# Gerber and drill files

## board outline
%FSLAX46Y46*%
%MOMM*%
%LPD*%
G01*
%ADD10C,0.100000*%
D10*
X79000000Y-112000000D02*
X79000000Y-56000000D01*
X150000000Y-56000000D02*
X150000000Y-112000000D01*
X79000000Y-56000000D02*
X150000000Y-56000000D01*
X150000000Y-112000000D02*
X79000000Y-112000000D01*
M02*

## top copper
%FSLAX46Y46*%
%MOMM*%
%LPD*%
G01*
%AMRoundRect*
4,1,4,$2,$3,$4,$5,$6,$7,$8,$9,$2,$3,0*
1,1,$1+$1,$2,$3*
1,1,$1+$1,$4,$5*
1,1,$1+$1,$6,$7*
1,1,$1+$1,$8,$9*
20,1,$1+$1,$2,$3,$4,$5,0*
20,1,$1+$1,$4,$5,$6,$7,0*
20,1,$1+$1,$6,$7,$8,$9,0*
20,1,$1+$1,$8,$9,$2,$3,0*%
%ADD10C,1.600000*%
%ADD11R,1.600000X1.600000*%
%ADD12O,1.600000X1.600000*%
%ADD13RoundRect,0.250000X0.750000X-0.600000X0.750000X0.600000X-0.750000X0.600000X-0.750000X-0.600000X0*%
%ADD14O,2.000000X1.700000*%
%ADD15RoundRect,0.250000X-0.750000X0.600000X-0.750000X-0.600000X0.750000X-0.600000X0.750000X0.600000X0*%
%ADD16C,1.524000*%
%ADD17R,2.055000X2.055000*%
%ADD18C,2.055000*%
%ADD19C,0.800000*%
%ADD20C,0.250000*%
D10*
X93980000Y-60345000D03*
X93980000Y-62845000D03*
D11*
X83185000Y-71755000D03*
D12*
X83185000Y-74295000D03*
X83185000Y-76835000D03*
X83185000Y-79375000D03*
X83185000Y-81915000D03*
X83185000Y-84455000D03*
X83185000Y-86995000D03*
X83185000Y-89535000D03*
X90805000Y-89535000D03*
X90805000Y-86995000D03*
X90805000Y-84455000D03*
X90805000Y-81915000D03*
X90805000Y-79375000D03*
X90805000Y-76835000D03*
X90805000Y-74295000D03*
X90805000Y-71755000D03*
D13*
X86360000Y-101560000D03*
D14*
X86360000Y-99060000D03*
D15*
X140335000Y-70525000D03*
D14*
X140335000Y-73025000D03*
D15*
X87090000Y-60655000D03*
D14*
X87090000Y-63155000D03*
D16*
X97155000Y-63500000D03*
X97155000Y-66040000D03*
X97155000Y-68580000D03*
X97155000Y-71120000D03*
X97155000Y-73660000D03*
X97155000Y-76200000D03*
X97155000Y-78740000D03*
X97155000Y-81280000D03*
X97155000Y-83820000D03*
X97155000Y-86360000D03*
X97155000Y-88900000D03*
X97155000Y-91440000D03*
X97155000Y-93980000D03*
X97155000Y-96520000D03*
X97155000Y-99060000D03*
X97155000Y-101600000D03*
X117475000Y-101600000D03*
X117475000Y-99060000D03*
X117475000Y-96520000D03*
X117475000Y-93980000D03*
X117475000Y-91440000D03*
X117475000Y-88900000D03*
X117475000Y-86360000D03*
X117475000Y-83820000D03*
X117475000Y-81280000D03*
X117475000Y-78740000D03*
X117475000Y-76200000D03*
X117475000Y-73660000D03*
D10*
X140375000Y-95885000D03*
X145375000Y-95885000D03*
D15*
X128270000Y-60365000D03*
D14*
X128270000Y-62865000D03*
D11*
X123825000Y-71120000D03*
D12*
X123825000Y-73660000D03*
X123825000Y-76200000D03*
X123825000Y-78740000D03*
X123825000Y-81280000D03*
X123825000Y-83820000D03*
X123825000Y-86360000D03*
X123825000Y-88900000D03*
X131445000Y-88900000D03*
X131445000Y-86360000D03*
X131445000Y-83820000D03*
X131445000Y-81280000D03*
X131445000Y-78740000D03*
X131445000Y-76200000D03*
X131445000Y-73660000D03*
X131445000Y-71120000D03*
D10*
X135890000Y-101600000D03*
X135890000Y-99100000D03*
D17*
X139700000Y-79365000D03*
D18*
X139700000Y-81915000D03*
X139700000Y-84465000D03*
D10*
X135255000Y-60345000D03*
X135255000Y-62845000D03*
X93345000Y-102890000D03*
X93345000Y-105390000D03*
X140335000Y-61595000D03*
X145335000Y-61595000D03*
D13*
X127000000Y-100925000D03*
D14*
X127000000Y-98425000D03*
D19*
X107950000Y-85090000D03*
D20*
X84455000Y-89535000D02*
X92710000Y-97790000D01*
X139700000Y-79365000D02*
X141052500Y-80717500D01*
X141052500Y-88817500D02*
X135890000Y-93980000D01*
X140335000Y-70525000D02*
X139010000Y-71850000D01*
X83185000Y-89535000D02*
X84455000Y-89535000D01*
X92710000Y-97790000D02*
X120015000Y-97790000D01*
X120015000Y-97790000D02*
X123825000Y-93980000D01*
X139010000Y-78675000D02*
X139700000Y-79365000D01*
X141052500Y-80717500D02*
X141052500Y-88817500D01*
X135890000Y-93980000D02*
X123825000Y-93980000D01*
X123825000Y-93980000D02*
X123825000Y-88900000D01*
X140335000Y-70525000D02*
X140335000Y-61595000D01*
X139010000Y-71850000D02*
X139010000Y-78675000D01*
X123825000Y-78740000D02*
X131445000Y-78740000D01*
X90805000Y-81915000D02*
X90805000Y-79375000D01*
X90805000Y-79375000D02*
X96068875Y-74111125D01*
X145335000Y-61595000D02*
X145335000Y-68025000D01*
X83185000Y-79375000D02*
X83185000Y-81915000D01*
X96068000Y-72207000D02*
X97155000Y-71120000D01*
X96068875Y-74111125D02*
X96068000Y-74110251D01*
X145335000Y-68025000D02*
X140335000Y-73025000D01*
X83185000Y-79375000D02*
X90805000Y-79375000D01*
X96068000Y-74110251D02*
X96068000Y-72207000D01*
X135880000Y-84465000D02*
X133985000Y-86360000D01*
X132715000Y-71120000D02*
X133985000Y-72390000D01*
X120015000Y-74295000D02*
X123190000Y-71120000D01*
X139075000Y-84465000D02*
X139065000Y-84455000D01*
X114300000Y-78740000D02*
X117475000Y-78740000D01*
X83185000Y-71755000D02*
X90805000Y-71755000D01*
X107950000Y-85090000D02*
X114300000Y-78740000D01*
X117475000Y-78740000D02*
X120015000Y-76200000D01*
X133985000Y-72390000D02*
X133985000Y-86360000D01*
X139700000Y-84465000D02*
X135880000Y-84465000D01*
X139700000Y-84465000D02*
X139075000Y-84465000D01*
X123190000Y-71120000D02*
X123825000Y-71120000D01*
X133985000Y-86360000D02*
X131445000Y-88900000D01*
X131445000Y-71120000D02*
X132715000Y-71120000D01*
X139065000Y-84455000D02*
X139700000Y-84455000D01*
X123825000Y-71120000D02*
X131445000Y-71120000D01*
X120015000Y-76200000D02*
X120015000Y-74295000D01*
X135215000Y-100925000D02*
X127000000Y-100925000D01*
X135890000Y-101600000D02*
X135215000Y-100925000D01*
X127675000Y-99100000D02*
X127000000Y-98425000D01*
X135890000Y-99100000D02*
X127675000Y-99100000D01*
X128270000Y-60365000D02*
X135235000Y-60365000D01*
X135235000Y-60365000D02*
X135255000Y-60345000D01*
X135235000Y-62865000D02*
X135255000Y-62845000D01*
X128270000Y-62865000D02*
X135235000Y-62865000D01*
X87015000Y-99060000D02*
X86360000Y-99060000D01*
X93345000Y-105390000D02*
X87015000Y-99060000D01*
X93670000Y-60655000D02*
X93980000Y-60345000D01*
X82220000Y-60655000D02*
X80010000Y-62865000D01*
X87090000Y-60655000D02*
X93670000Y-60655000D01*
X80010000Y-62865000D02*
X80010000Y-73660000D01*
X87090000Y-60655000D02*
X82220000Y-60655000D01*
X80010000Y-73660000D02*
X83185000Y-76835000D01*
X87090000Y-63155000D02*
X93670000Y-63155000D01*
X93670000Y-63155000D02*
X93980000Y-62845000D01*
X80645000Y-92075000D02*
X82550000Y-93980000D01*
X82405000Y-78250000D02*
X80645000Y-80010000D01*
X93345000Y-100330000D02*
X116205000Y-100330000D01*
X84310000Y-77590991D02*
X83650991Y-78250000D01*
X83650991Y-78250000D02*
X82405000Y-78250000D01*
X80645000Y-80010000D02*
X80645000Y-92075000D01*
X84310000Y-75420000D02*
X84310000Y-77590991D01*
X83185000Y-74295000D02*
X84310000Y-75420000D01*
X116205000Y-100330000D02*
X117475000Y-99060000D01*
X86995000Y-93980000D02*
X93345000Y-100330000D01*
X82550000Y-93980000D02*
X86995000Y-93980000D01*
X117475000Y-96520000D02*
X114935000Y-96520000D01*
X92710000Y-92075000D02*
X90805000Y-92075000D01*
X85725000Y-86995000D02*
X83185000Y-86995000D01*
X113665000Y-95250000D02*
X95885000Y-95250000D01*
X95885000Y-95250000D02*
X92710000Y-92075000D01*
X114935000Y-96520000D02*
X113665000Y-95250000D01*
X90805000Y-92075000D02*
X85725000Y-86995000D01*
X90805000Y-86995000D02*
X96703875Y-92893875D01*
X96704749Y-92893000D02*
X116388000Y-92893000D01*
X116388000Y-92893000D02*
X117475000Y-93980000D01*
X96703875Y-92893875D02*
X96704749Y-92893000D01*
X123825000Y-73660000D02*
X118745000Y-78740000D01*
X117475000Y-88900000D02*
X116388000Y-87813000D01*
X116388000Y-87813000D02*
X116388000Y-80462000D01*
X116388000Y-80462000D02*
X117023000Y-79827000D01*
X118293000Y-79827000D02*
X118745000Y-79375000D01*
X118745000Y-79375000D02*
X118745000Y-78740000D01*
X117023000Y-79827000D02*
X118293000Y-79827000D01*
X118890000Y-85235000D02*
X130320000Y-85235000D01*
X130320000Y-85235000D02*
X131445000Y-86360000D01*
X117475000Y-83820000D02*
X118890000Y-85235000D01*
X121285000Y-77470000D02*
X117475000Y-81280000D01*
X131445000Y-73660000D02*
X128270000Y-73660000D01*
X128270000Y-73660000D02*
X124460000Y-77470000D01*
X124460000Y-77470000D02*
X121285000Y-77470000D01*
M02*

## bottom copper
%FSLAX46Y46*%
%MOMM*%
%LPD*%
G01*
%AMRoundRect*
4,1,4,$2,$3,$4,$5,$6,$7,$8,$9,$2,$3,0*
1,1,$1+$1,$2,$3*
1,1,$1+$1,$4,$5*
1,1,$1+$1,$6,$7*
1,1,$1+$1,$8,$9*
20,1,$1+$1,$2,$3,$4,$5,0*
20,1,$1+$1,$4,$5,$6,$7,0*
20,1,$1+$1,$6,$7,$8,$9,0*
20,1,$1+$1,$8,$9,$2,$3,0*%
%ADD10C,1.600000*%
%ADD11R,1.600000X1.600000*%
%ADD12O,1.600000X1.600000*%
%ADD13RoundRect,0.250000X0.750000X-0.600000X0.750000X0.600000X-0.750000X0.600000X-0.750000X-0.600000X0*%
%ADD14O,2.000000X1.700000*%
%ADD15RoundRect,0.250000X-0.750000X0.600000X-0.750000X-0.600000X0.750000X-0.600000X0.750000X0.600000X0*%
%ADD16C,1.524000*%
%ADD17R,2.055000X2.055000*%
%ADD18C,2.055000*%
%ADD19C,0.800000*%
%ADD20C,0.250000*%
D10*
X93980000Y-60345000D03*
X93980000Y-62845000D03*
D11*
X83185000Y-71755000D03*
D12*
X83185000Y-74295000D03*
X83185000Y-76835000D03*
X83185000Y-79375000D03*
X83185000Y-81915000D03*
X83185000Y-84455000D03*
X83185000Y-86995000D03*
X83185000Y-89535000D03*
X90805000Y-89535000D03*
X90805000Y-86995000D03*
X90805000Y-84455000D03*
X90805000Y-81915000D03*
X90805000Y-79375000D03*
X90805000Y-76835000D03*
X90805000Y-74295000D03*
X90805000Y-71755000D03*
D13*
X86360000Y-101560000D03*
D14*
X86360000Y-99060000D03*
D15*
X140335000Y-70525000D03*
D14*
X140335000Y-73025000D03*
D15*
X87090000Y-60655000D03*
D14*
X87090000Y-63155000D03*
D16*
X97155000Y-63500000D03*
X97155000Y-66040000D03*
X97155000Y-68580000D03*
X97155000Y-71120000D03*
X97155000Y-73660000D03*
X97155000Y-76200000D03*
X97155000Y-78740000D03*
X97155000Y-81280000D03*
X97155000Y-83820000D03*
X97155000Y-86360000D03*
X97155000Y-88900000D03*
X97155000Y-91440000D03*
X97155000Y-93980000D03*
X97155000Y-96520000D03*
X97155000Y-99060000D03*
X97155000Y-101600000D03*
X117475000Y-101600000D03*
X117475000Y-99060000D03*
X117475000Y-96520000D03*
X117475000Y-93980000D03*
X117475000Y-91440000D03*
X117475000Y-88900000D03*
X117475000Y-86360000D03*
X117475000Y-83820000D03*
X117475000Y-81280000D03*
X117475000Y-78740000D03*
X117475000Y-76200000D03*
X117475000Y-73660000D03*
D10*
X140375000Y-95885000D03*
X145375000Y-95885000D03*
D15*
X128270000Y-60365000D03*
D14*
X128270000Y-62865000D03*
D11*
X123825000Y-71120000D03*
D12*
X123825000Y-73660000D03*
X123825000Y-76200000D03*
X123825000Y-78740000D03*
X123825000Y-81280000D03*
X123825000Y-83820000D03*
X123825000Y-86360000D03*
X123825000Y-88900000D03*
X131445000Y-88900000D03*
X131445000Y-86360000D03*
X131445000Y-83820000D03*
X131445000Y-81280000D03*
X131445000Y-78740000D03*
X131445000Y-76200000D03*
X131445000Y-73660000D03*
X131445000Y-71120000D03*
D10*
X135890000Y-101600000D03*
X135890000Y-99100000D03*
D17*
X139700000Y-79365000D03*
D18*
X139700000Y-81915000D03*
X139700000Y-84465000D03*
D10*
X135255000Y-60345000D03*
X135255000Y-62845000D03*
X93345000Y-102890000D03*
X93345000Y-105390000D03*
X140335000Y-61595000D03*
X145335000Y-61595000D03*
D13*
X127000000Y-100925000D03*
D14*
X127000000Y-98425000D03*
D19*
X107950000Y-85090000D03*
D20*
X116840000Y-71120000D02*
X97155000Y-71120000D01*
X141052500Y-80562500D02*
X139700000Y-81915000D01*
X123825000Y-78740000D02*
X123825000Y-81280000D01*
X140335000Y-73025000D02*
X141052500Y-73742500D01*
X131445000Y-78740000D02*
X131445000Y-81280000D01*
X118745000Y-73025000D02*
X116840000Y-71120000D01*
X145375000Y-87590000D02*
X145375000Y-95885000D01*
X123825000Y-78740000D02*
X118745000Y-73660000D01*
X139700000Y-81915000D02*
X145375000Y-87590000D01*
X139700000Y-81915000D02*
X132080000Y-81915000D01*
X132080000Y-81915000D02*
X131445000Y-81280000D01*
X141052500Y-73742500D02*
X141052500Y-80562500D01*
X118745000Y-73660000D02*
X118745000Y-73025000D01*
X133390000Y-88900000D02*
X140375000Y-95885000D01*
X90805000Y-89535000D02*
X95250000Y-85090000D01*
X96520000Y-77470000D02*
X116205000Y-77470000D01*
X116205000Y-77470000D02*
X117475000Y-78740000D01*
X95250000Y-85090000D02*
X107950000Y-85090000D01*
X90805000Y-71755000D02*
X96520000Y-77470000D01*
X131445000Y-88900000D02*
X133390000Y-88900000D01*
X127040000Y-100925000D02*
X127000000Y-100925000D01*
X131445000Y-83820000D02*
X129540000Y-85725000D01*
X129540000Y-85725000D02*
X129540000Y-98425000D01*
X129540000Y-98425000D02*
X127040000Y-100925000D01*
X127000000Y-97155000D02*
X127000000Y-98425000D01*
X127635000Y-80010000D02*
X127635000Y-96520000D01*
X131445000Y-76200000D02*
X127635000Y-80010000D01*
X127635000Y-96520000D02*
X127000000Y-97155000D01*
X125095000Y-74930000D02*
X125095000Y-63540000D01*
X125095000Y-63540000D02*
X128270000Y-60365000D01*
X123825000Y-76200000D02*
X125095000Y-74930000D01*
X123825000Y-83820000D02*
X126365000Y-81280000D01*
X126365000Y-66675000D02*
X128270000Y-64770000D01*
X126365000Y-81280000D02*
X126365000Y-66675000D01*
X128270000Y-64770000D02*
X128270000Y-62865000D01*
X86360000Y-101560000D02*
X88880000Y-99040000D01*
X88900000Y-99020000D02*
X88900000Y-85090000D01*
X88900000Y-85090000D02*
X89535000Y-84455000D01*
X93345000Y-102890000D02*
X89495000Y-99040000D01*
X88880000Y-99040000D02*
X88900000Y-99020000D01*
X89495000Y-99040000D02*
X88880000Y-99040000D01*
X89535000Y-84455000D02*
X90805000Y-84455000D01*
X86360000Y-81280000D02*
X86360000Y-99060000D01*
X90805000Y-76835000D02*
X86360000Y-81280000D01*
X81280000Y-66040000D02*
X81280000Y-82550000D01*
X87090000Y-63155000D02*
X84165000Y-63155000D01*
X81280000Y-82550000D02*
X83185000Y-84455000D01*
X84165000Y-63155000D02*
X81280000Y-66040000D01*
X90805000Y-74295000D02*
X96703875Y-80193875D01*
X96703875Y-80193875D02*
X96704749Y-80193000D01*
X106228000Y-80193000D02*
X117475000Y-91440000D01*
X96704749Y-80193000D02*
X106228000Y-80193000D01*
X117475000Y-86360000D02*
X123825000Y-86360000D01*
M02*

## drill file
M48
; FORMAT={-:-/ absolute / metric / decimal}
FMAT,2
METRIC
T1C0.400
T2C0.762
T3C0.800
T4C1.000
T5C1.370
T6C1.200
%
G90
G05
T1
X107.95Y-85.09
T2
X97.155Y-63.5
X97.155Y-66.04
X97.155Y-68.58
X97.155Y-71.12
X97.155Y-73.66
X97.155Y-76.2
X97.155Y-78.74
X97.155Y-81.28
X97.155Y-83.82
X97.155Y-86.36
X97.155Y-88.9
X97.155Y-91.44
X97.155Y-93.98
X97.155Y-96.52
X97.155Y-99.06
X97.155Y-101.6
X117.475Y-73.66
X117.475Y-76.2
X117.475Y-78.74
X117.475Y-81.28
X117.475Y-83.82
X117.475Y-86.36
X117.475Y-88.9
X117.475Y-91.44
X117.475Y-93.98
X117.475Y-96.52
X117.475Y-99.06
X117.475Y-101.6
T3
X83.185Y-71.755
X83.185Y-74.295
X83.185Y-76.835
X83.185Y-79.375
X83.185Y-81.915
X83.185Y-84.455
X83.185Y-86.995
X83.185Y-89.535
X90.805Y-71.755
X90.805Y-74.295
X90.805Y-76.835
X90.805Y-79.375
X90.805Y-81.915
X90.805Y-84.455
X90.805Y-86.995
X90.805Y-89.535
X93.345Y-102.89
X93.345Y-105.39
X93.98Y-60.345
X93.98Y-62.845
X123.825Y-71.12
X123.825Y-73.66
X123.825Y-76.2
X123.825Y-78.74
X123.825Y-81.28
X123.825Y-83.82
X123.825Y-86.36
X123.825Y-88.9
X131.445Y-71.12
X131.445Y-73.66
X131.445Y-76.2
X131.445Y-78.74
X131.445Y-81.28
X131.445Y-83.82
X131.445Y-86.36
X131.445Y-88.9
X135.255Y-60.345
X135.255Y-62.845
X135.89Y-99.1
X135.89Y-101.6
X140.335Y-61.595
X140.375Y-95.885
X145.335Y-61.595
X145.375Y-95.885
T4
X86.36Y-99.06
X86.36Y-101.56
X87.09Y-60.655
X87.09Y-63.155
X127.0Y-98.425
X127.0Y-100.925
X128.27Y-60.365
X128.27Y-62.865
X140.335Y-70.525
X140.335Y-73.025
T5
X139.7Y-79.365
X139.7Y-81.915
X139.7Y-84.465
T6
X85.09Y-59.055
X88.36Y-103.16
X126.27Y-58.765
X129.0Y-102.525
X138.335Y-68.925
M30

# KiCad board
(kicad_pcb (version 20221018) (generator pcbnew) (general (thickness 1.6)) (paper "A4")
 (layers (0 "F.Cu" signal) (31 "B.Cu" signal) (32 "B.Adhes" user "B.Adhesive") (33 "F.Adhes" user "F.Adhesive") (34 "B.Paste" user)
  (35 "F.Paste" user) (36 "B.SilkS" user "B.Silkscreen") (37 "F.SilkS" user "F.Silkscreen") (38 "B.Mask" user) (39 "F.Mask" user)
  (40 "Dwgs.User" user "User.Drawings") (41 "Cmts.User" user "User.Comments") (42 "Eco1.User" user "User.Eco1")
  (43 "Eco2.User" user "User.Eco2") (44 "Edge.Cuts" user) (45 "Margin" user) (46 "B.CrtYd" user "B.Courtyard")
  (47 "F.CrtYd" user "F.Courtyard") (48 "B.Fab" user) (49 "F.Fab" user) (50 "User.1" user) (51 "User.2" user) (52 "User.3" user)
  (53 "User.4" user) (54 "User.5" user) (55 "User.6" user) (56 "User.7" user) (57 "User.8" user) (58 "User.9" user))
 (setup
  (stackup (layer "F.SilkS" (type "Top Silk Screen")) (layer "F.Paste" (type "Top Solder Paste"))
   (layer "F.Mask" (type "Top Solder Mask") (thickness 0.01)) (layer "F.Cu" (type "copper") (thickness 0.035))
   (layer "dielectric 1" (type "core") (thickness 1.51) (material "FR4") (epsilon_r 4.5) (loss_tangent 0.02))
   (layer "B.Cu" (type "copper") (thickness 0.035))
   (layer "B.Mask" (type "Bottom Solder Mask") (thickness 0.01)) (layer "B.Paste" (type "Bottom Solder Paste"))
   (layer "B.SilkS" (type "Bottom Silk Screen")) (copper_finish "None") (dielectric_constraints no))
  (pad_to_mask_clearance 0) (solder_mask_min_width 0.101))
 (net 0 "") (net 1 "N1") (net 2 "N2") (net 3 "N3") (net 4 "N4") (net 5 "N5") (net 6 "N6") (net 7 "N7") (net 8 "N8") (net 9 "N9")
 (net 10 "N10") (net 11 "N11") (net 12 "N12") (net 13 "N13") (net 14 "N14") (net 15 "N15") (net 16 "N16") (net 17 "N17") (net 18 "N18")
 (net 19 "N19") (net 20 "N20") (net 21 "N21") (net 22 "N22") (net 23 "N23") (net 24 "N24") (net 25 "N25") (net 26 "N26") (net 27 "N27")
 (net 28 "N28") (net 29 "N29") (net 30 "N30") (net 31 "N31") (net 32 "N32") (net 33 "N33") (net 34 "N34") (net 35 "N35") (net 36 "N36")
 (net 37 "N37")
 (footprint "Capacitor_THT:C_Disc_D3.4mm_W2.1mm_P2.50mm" (layer "F.Cu") (at 93.98 60.345 -90)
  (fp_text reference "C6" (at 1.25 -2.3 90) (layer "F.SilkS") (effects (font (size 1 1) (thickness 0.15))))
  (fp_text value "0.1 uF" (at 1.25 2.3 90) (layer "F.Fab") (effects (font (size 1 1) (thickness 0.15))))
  (pad "1" thru_hole circle (at 0 0 270) (size 1.6 1.6) (drill 0.8) (layers "*.Cu" "*.Mask") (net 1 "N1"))
  (pad "2" thru_hole circle (at 2.5 0 270) (size 1.6 1.6) (drill 0.8) (layers "*.Cu" "*.Mask") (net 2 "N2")))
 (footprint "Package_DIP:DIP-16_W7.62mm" (layer "F.Cu") (at 83.185 71.755)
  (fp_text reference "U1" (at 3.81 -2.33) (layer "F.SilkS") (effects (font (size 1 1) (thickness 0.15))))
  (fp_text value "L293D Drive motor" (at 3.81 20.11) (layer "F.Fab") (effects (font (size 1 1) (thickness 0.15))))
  (pad "1" thru_hole rect (at 0 0) (size 1.6 1.6) (drill 0.8) (layers "*.Cu" "*.Mask") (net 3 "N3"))
  (pad "2" thru_hole oval (at 0 2.54) (size 1.6 1.6) (drill 0.8) (layers "*.Cu" "*.Mask") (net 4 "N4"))
  (pad "3" thru_hole oval (at 0 5.08) (size 1.6 1.6) (drill 0.8) (layers "*.Cu" "*.Mask") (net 1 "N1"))
  (pad "4" thru_hole oval (at 0 7.62) (size 1.6 1.6) (drill 0.8) (layers "*.Cu" "*.Mask") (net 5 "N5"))
  (pad "5" thru_hole oval (at 0 10.16) (size 1.6 1.6) (drill 0.8) (layers "*.Cu" "*.Mask") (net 5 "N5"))
  (pad "6" thru_hole oval (at 0 12.7) (size 1.6 1.6) (drill 0.8) (layers "*.Cu" "*.Mask") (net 2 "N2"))
  (pad "7" thru_hole oval (at 0 15.24) (size 1.6 1.6) (drill 0.8) (layers "*.Cu" "*.Mask") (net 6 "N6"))
  (pad "8" thru_hole oval (at 0 17.78) (size 1.6 1.6) (drill 0.8) (layers "*.Cu" "*.Mask") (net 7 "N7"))
  (pad "9" thru_hole oval (at 7.62 17.78) (size 1.6 1.6) (drill 0.8) (layers "*.Cu" "*.Mask") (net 3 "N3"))
  (pad "10" thru_hole oval (at 7.62 15.24) (size 1.6 1.6) (drill 0.8) (layers "*.Cu" "*.Mask") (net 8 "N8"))
  (pad "11" thru_hole oval (at 7.62 12.7) (size 1.6 1.6) (drill 0.8) (layers "*.Cu" "*.Mask") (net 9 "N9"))
  (pad "12" thru_hole oval (at 7.62 10.16) (size 1.6 1.6) (drill 0.8) (layers "*.Cu" "*.Mask") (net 5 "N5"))
  (pad "13" thru_hole oval (at 7.62 7.62) (size 1.6 1.6) (drill 0.8) (layers "*.Cu" "*.Mask") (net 5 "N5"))
  (pad "14" thru_hole oval (at 7.62 5.08) (size 1.6 1.6) (drill 0.8) (layers "*.Cu" "*.Mask") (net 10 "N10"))
  (pad "15" thru_hole oval (at 7.62 2.54) (size 1.6 1.6) (drill 0.8) (layers "*.Cu" "*.Mask") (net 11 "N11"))
  (pad "16" thru_hole oval (at 7.62 0) (size 1.6 1.6) (drill 0.8) (layers "*.Cu" "*.Mask") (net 3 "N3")))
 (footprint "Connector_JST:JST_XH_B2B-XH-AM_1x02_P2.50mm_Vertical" (layer "F.Cu") (at 86.36 101.56 90)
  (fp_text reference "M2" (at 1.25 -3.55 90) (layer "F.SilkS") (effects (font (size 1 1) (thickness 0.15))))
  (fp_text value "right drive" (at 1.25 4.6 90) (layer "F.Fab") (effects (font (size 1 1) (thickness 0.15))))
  (pad "" np_thru_hole circle (at -1.6 2 90) (size 1.2 1.2) (drill 1.2) (layers "*.Cu" "*.Mask"))
  (pad "1" thru_hole roundrect (at 0 0 90) (size 1.7 2) (drill 1) (layers "*.Cu" "*.Mask") (roundrect_rratio 0.147059) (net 9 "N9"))
  (pad "2" thru_hole oval (at 2.5 0 90) (size 1.7 2) (drill 1) (layers "*.Cu" "*.Mask") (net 10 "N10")))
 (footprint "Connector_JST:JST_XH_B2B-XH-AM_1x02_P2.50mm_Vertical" (layer "F.Cu") (at 140.335 70.525 -90)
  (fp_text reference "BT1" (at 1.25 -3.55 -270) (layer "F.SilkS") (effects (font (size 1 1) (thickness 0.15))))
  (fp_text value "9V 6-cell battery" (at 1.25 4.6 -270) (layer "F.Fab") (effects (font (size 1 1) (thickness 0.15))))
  (pad "" np_thru_hole circle (at -1.6 2 270) (size 1.2 1.2) (drill 1.2) (layers "*.Cu" "*.Mask"))
  (pad "1" thru_hole roundrect (at 0 0 270) (size 1.7 2) (drill 1) (layers "*.Cu" "*.Mask") (roundrect_rratio 0.147059) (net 7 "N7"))
  (pad "2" thru_hole oval (at 2.5 0 270) (size 1.7 2) (drill 1) (layers "*.Cu" "*.Mask") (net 5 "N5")))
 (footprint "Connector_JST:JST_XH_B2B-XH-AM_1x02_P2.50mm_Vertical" (layer "F.Cu") (at 87.09 60.655 -90)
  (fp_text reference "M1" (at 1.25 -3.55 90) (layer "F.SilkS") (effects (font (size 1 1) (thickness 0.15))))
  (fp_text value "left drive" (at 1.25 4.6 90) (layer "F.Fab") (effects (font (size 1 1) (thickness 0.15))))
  (pad "" np_thru_hole circle (at -1.6 2 270) (size 1.2 1.2) (drill 1.2) (layers "*.Cu" "*.Mask"))
  (pad "1" thru_hole roundrect (at 0 0 270) (size 1.7 2) (drill 1) (layers "*.Cu" "*.Mask") (roundrect_rratio 0.147059) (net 1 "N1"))
  (pad "2" thru_hole oval (at 2.5 0 270) (size 1.7 2) (drill 1) (layers "*.Cu" "*.Mask") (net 2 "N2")))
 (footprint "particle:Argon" (layer "F.Cu") (at 107.315 82.55)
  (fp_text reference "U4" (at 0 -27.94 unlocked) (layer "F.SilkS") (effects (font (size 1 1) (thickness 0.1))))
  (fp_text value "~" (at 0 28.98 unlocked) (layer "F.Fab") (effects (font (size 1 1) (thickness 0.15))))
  (pad "1" thru_hole circle (at -10.16 -19.05) (size 1.524 1.524) (drill 0.762) (layers "*.Cu" "*.Mask") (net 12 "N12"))
  (pad "2" thru_hole circle (at -10.16 -16.51) (size 1.524 1.524) (drill 0.762) (layers "*.Cu" "*.Mask") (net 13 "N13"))
  (pad "3" thru_hole circle (at -10.16 -13.97) (size 1.524 1.524) (drill 0.762) (layers "*.Cu" "*.Mask") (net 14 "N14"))
  (pad "4" thru_hole circle (at -10.16 -11.43) (size 1.524 1.524) (drill 0.762) (layers "*.Cu" "*.Mask") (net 5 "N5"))
  (pad "5" thru_hole circle (at -10.16 -8.89) (size 1.524 1.524) (drill 0.762) (layers "*.Cu" "*.Mask") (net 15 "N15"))
  (pad "6" thru_hole circle (at -10.16 -6.35) (size 1.524 1.524) (drill 0.762) (layers "*.Cu" "*.Mask") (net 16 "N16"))
  (pad "7" thru_hole circle (at -10.16 -3.81) (size 1.524 1.524) (drill 0.762) (layers "*.Cu" "*.Mask") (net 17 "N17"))
  (pad "8" thru_hole circle (at -10.16 -1.27) (size 1.524 1.524) (drill 0.762) (layers "*.Cu" "*.Mask") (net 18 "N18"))
  (pad "9" thru_hole circle (at -10.16 1.27) (size 1.524 1.524) (drill 0.762) (layers "*.Cu" "*.Mask") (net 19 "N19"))
  (pad "10" thru_hole circle (at -10.16 3.81) (size 1.524 1.524) (drill 0.762) (layers "*.Cu" "*.Mask") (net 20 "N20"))
  (pad "11" thru_hole circle (at -10.16 6.35) (size 1.524 1.524) (drill 0.762) (layers "*.Cu" "*.Mask") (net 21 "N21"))
  (pad "12" thru_hole circle (at -10.16 8.89) (size 1.524 1.524) (drill 0.762) (layers "*.Cu" "*.Mask") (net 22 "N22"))
  (pad "13" thru_hole circle (at -10.16 11.43) (size 1.524 1.524) (drill 0.762) (layers "*.Cu" "*.Mask") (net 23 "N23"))
  (pad "14" thru_hole circle (at -10.16 13.97) (size 1.524 1.524) (drill 0.762) (layers "*.Cu" "*.Mask") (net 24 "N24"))
  (pad "15" thru_hole circle (at -10.16 16.51) (size 1.524 1.524) (drill 0.762) (layers "*.Cu" "*.Mask") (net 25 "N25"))
  (pad "16" thru_hole circle (at -10.16 19.05) (size 1.524 1.524) (drill 0.762) (layers "*.Cu" "*.Mask") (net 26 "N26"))
  (pad "17" thru_hole circle (at 10.16 19.05) (size 1.524 1.524) (drill 0.762) (layers "*.Cu" "*.Mask") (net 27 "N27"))
  (pad "18" thru_hole circle (at 10.16 16.51) (size 1.524 1.524) (drill 0.762) (layers "*.Cu" "*.Mask") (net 4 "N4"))
  (pad "19" thru_hole circle (at 10.16 13.97) (size 1.524 1.524) (drill 0.762) (layers "*.Cu" "*.Mask") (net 6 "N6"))
  (pad "20" thru_hole circle (at 10.16 11.43) (size 1.524 1.524) (drill 0.762) (layers "*.Cu" "*.Mask") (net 8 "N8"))
  (pad "21" thru_hole circle (at 10.16 8.89) (size 1.524 1.524) (drill 0.762) (layers "*.Cu" "*.Mask") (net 11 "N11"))
  (pad "22" thru_hole circle (at 10.16 6.35) (size 1.524 1.524) (drill 0.762) (layers "*.Cu" "*.Mask") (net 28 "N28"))
  (pad "23" thru_hole circle (at 10.16 3.81) (size 1.524 1.524) (drill 0.762) (layers "*.Cu" "*.Mask") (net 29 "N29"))
  (pad "24" thru_hole circle (at 10.16 1.27) (size 1.524 1.524) (drill 0.762) (layers "*.Cu" "*.Mask") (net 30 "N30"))
  (pad "25" thru_hole circle (at 10.16 -1.27) (size 1.524 1.524) (drill 0.762) (layers "*.Cu" "*.Mask") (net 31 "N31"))
  (pad "26" thru_hole circle (at 10.16 -3.81) (size 1.524 1.524) (drill 0.762) (layers "*.Cu" "*.Mask") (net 3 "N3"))
  (pad "27" thru_hole circle (at 10.16 -6.35) (size 1.524 1.524) (drill 0.762) (layers "*.Cu" "*.Mask") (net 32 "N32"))
  (pad "28" thru_hole circle (at 10.16 -8.89) (size 1.524 1.524) (drill 0.762) (layers "*.Cu" "*.Mask") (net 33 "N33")))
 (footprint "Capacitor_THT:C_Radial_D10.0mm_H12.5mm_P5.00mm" (layer "F.Cu") (at 140.375 95.885)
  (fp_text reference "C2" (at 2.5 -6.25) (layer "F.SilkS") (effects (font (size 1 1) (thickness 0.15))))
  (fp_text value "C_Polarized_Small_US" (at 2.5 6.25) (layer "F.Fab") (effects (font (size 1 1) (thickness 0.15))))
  (pad "1" thru_hole circle (at 0 0) (size 1.6 1.6) (drill 0.8) (layers "*.Cu" "*.Mask") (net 3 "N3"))
  (pad "2" thru_hole circle (at 5 0) (size 1.6 1.6) (drill 0.8) (layers "*.Cu" "*.Mask") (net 5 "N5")))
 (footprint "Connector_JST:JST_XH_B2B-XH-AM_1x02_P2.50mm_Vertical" (layer "F.Cu") (at 128.27 60.365 -90)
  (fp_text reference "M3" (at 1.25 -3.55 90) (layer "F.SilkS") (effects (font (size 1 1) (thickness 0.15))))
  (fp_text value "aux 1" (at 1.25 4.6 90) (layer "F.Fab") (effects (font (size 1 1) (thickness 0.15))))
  (pad "" np_thru_hole circle (at -1.6 2 270) (size 1.2 1.2) (drill 1.2) (layers "*.Cu" "*.Mask"))
  (pad "1" thru_hole roundrect (at 0 0 270) (size 1.7 2) (drill 1) (layers "*.Cu" "*.Mask") (roundrect_rratio 0.147059) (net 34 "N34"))
  (pad "2" thru_hole oval (at 2.5 0 270) (size 1.7 2) (drill 1) (layers "*.Cu" "*.Mask") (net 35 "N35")))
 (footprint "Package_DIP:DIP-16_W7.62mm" (layer "F.Cu") (at 123.825 71.12)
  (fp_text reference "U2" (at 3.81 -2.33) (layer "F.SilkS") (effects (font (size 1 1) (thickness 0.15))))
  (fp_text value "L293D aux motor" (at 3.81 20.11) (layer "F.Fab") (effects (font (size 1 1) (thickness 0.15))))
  (pad "1" thru_hole rect (at 0 0) (size 1.6 1.6) (drill 0.8) (layers "*.Cu" "*.Mask") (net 3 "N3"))
  (pad "2" thru_hole oval (at 0 2.54) (size 1.6 1.6) (drill 0.8) (layers "*.Cu" "*.Mask") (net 28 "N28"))
  (pad "3" thru_hole oval (at 0 5.08) (size 1.6 1.6) (drill 0.8) (layers "*.Cu" "*.Mask") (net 34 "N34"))
  (pad "4" thru_hole oval (at 0 7.62) (size 1.6 1.6) (drill 0.8) (layers "*.Cu" "*.Mask") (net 5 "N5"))
  (pad "5" thru_hole oval (at 0 10.16) (size 1.6 1.6) (drill 0.8) (layers "*.Cu" "*.Mask") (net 5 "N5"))
  (pad "6" thru_hole oval (at 0 12.7) (size 1.6 1.6) (drill 0.8) (layers "*.Cu" "*.Mask") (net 35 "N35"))
  (pad "7" thru_hole oval (at 0 15.24) (size 1.6 1.6) (drill 0.8) (layers "*.Cu" "*.Mask") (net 29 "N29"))
  (pad "8" thru_hole oval (at 0 17.78) (size 1.6 1.6) (drill 0.8) (layers "*.Cu" "*.Mask") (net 7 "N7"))
  (pad "9" thru_hole oval (at 7.62 17.78) (size 1.6 1.6) (drill 0.8) (layers "*.Cu" "*.Mask") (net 3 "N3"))
  (pad "10" thru_hole oval (at 7.62 15.24) (size 1.6 1.6) (drill 0.8) (layers "*.Cu" "*.Mask") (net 30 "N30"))
  (pad "11" thru_hole oval (at 7.62 12.7) (size 1.6 1.6) (drill 0.8) (layers "*.Cu" "*.Mask") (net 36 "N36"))
  (pad "12" thru_hole oval (at 7.62 10.16) (size 1.6 1.6) (drill 0.8) (layers "*.Cu" "*.Mask") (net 5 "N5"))
  (pad "13" thru_hole oval (at 7.62 7.62) (size 1.6 1.6) (drill 0.8) (layers "*.Cu" "*.Mask") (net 5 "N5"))
  (pad "14" thru_hole oval (at 7.62 5.08) (size 1.6 1.6) (drill 0.8) (layers "*.Cu" "*.Mask") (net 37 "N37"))
  (pad "15" thru_hole oval (at 7.62 2.54) (size 1.6 1.6) (drill 0.8) (layers "*.Cu" "*.Mask") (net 31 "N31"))
  (pad "16" thru_hole oval (at 7.62 0) (size 1.6 1.6) (drill 0.8) (layers "*.Cu" "*.Mask") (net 3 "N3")))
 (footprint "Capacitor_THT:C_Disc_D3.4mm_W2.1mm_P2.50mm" (layer "F.Cu") (at 135.89 101.6 90)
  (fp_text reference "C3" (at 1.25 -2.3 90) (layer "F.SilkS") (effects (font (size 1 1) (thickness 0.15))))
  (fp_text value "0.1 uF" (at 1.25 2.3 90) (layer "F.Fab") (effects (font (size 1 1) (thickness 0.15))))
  (pad "1" thru_hole circle (at 0 0 90) (size 1.6 1.6) (drill 0.8) (layers "*.Cu" "*.Mask") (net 36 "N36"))
  (pad "2" thru_hole circle (at 2.5 0 90) (size 1.6 1.6) (drill 0.8) (layers "*.Cu" "*.Mask") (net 37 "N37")))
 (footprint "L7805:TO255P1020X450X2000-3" (layer "F.Cu") (at 140.3625 81.915 -90)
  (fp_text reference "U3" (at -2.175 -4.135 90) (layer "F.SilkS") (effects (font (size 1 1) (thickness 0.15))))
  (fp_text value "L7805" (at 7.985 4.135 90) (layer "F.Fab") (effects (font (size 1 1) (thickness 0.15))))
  (pad "1" thru_hole rect (at -2.55 0.6625 270) (size 2.055 2.055) (drill 1.37) (layers "*.Cu" "*.Mask") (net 7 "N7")
   (solder_mask_margin 0.102))
  (pad "2" thru_hole circle (at 0 0.6625 270) (size 2.055 2.055) (drill 1.37) (layers "*.Cu" "*.Mask") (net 5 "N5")
   (solder_mask_margin 0.102))
  (pad "3" thru_hole circle (at 2.55 0.6625 270) (size 2.055 2.055) (drill 1.37) (layers "*.Cu" "*.Mask") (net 3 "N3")
   (solder_mask_margin 0.102)))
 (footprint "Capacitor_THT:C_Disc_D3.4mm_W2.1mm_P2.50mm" (layer "F.Cu") (at 135.255 60.345 -90)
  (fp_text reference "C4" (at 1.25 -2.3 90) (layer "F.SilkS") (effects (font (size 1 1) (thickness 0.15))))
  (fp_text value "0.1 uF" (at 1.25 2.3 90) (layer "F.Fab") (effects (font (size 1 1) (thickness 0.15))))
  (pad "1" thru_hole circle (at 0 0 270) (size 1.6 1.6) (drill 0.8) (layers "*.Cu" "*.Mask") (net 34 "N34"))
  (pad "2" thru_hole circle (at 2.5 0 270) (size 1.6 1.6) (drill 0.8) (layers "*.Cu" "*.Mask") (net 35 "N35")))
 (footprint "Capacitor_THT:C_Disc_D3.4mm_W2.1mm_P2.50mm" (layer "F.Cu") (at 93.345 102.89 -90)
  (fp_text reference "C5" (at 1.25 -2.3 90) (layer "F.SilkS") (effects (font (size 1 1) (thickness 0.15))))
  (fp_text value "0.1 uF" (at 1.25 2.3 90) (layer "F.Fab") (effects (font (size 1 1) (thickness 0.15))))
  (pad "1" thru_hole circle (at 0 0 270) (size 1.6 1.6) (drill 0.8) (layers "*.Cu" "*.Mask") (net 9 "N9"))
  (pad "2" thru_hole circle (at 2.5 0 270) (size 1.6 1.6) (drill 0.8) (layers "*.Cu" "*.Mask") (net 10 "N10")))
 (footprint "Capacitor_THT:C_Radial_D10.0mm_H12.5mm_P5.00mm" (layer "F.Cu") (at 140.335 61.595)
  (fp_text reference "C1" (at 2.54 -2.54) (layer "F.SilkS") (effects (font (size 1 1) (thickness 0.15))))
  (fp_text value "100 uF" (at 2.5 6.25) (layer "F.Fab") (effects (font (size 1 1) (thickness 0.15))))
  (pad "1" thru_hole circle (at 0 0) (size 1.6 1.6) (drill 0.8) (layers "*.Cu" "*.Mask") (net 7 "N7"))
  (pad "2" thru_hole circle (at 5 0) (size 1.6 1.6) (drill 0.8) (layers "*.Cu" "*.Mask") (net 5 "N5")))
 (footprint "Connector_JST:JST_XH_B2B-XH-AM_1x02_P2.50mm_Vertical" (layer "F.Cu") (at 127 100.925 90)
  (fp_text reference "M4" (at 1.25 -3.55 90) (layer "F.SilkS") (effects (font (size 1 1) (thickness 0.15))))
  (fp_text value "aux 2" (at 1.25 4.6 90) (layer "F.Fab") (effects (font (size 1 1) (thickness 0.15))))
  (pad "" np_thru_hole circle (at -1.6 2 90) (size 1.2 1.2) (drill 1.2) (layers "*.Cu" "*.Mask"))
  (pad "1" thru_hole roundrect (at 0 0 90) (size 1.7 2) (drill 1) (layers "*.Cu" "*.Mask") (roundrect_rratio 0.147059) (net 36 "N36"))
  (pad "2" thru_hole oval (at 2.5 0 90) (size 1.7 2) (drill 1) (layers "*.Cu" "*.Mask") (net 37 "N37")))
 (gr_line (start 79 112) (end 79 56) (stroke (width 0.1) (type default)) (layer "Edge.Cuts"))
 (gr_line (start 150 56) (end 150 112) (stroke (width 0.1) (type default)) (layer "Edge.Cuts"))
 (gr_line (start 79 56) (end 150 56) (stroke (width 0.1) (type default)) (layer "Edge.Cuts"))
 (gr_line (start 150 112) (end 79 112) (stroke (width 0.1) (type default)) (layer "Edge.Cuts"))
 (segment (start 84.455 89.535) (end 92.71 97.79) (width 0.25) (layer "F.Cu") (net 7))
 (segment (start 139.7 79.365) (end 141.0525 80.7175) (width 0.25) (layer "F.Cu") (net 7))
 (segment (start 141.0525 88.8175) (end 135.89 93.98) (width 0.25) (layer "F.Cu") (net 7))
 (segment (start 140.335 70.525) (end 139.01 71.85) (width 0.25) (layer "F.Cu") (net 7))
 (segment (start 83.185 89.535) (end 84.455 89.535) (width 0.25) (layer "F.Cu") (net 7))
 (segment (start 92.71 97.79) (end 120.015 97.79) (width 0.25) (layer "F.Cu") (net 7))
 (segment (start 120.015 97.79) (end 123.825 93.98) (width 0.25) (layer "F.Cu") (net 7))
 (segment (start 139.01 78.675) (end 139.7 79.365) (width 0.25) (layer "F.Cu") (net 7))
 (segment (start 141.0525 80.7175) (end 141.0525 88.8175) (width 0.25) (layer "F.Cu") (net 7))
 (segment (start 135.89 93.98) (end 123.825 93.98) (width 0.25) (layer "F.Cu") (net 7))
 (segment (start 123.825 93.98) (end 123.825 88.9) (width 0.25) (layer "F.Cu") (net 7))
 (segment (start 140.335 70.525) (end 140.335 61.595) (width 0.25) (layer "F.Cu") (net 7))
 (segment (start 139.01 71.85) (end 139.01 78.675) (width 0.25) (layer "F.Cu") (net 7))
 (segment (start 123.825 78.74) (end 131.445 78.74) (width 0.25) (layer "F.Cu") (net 5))
 (segment (start 90.805 81.915) (end 90.805 79.375) (width 0.25) (layer "F.Cu") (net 5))
 (segment (start 90.805 79.375) (end 96.068875 74.111125) (width 0.25) (layer "F.Cu") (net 5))
 (segment (start 145.335 61.595) (end 145.335 68.025) (width 0.25) (layer "F.Cu") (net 5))
 (segment (start 83.185 79.375) (end 83.185 81.915) (width 0.25) (layer "F.Cu") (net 5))
 (segment (start 96.068 72.207) (end 97.155 71.12) (width 0.25) (layer "F.Cu") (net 5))
 (segment (start 96.068875 74.111125) (end 96.068 74.110251) (width 0.25) (layer "F.Cu") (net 5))
 (segment (start 145.335 68.025) (end 140.335 73.025) (width 0.25) (layer "F.Cu") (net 5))
 (segment (start 83.185 79.375) (end 90.805 79.375) (width 0.25) (layer "F.Cu") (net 5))
 (segment (start 96.068 74.110251) (end 96.068 72.207) (width 0.25) (layer "F.Cu") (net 5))
 (segment (start 116.84 71.12) (end 97.155 71.12) (width 0.25) (layer "B.Cu") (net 5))
 (segment (start 141.0525 80.5625) (end 139.7 81.915) (width 0.25) (layer "B.Cu") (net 5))
 (segment (start 123.825 78.74) (end 123.825 81.28) (width 0.25) (layer "B.Cu") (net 5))
 (segment (start 140.335 73.025) (end 141.0525 73.7425) (width 0.25) (layer "B.Cu") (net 5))
 (segment (start 131.445 78.74) (end 131.445 81.28) (width 0.25) (layer "B.Cu") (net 5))
 (segment (start 118.745 73.025) (end 116.84 71.12) (width 0.25) (layer "B.Cu") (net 5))
 (segment (start 145.375 87.59) (end 145.375 95.885) (width 0.25) (layer "B.Cu") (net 5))
 (segment (start 123.825 78.74) (end 118.745 73.66) (width 0.25) (layer "B.Cu") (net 5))
 (segment (start 139.7 81.915) (end 145.375 87.59) (width 0.25) (layer "B.Cu") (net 5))
 (segment (start 139.7 81.915) (end 132.08 81.915) (width 0.25) (layer "B.Cu") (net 5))
 (segment (start 132.08 81.915) (end 131.445 81.28) (width 0.25) (layer "B.Cu") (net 5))
 (segment (start 141.0525 73.7425) (end 141.0525 80.5625) (width 0.25) (layer "B.Cu") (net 5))
 (segment (start 118.745 73.66) (end 118.745 73.025) (width 0.25) (layer "B.Cu") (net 5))
 (segment (start 135.88 84.465) (end 133.985 86.36) (width 0.25) (layer "F.Cu") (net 3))
 (segment (start 132.715 71.12) (end 133.985 72.39) (width 0.25) (layer "F.Cu") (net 3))
 (segment (start 120.015 74.295) (end 123.19 71.12) (width 0.25) (layer "F.Cu") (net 3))
 (segment (start 139.075 84.465) (end 139.065 84.455) (width 0.25) (layer "F.Cu") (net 3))
 (segment (start 114.3 78.74) (end 117.475 78.74) (width 0.25) (layer "F.Cu") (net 3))
 (segment (start 83.185 71.755) (end 90.805 71.755) (width 0.25) (layer "F.Cu") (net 3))
 (segment (start 107.95 85.09) (end 114.3 78.74) (width 0.25) (layer "F.Cu") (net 3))
 (segment (start 117.475 78.74) (end 120.015 76.2) (width 0.25) (layer "F.Cu") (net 3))
 (segment (start 133.985 72.39) (end 133.985 86.36) (width 0.25) (layer "F.Cu") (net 3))
 (segment (start 139.7 84.465) (end 135.88 84.465) (width 0.25) (layer "F.Cu") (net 3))
 (segment (start 139.7 84.465) (end 139.075 84.465) (width 0.25) (layer "F.Cu") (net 3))
 (segment (start 123.19 71.12) (end 123.825 71.12) (width 0.25) (layer "F.Cu") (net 3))
 (segment (start 133.985 86.36) (end 131.445 88.9) (width 0.25) (layer "F.Cu") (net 3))
 (segment (start 131.445 71.12) (end 132.715 71.12) (width 0.25) (layer "F.Cu") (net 3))
 (segment (start 139.065 84.455) (end 139.7 84.455) (width 0.25) (layer "F.Cu") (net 3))
 (segment (start 123.825 71.12) (end 131.445 71.12) (width 0.25) (layer "F.Cu") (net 3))
 (segment (start 120.015 76.2) (end 120.015 74.295) (width 0.25) (layer "F.Cu") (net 3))
 (via (at 107.95 85.09) (size 0.8) (drill 0.4) (layers "F.Cu" "B.Cu") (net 3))
 (segment (start 133.39 88.9) (end 140.375 95.885) (width 0.25) (layer "B.Cu") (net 3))
 (segment (start 90.805 89.535) (end 95.25 85.09) (width 0.25) (layer "B.Cu") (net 3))
 (segment (start 96.52 77.47) (end 116.205 77.47) (width 0.25) (layer "B.Cu") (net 3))
 (segment (start 116.205 77.47) (end 117.475 78.74) (width 0.25) (layer "B.Cu") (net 3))
 (segment (start 95.25 85.09) (end 107.95 85.09) (width 0.25) (layer "B.Cu") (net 3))
 (segment (start 90.805 71.755) (end 96.52 77.47) (width 0.25) (layer "B.Cu") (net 3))
 (segment (start 131.445 88.9) (end 133.39 88.9) (width 0.25) (layer "B.Cu") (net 3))
 (segment (start 135.215 100.925) (end 127 100.925) (width 0.25) (layer "F.Cu") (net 36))
 (segment (start 135.89 101.6) (end 135.215 100.925) (width 0.25) (layer "F.Cu") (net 36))
 (segment (start 127.04 100.925) (end 127 100.925) (width 0.25) (layer "B.Cu") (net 36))
 (segment (start 131.445 83.82) (end 129.54 85.725) (width 0.25) (layer "B.Cu") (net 36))
 (segment (start 129.54 85.725) (end 129.54 98.425) (width 0.25) (layer "B.Cu") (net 36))
 (segment (start 129.54 98.425) (end 127.04 100.925) (width 0.25) (layer "B.Cu") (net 36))
 (segment (start 127.675 99.1) (end 127 98.425) (width 0.25) (layer "F.Cu") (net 37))
 (segment (start 135.89 99.1) (end 127.675 99.1) (width 0.25) (layer "F.Cu") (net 37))
 (segment (start 127 97.155) (end 127 98.425) (width 0.25) (layer "B.Cu") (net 37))
 (segment (start 127.635 80.01) (end 127.635 96.52) (width 0.25) (layer "B.Cu") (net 37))
 (segment (start 131.445 76.2) (end 127.635 80.01) (width 0.25) (layer "B.Cu") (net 37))
 (segment (start 127.635 96.52) (end 127 97.155) (width 0.25) (layer "B.Cu") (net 37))
 (segment (start 128.27 60.365) (end 135.235 60.365) (width 0.25) (layer "F.Cu") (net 34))
 (segment (start 135.235 60.365) (end 135.255 60.345) (width 0.25) (layer "F.Cu") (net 34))
 (segment (start 125.095 74.93) (end 125.095 63.54) (width 0.25) (layer "B.Cu") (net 34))
 (segment (start 125.095 63.54) (end 128.27 60.365) (width 0.25) (layer "B.Cu") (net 34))
 (segment (start 123.825 76.2) (end 125.095 74.93) (width 0.25) (layer "B.Cu") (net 34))
 (segment (start 135.235 62.865) (end 135.255 62.845) (width 0.25) (layer "F.Cu") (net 35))
 (segment (start 128.27 62.865) (end 135.235 62.865) (width 0.25) (layer "F.Cu") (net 35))
 (segment (start 123.825 83.82) (end 126.365 81.28) (width 0.25) (layer "B.Cu") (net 35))
 (segment (start 126.365 66.675) (end 128.27 64.77) (width 0.25) (layer "B.Cu") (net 35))
 (segment (start 126.365 81.28) (end 126.365 66.675) (width 0.25) (layer "B.Cu") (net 35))
 (segment (start 128.27 64.77) (end 128.27 62.865) (width 0.25) (layer "B.Cu") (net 35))
 (segment (start 86.36 101.56) (end 88.88 99.04) (width 0.25) (layer "B.Cu") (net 9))
 (segment (start 88.9 99.02) (end 88.9 85.09) (width 0.25) (layer "B.Cu") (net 9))
 (segment (start 88.9 85.09) (end 89.535 84.455) (width 0.25) (layer "B.Cu") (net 9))
 (segment (start 93.345 102.89) (end 89.495 99.04) (width 0.25) (layer "B.Cu") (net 9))
 (segment (start 88.88 99.04) (end 88.9 99.02) (width 0.25) (layer "B.Cu") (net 9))
 (segment (start 89.495 99.04) (end 88.88 99.04) (width 0.25) (layer "B.Cu") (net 9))
 (segment (start 89.535 84.455) (end 90.805 84.455) (width 0.25) (layer "B.Cu") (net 9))
 (segment (start 87.015 99.06) (end 86.36 99.06) (width 0.25) (layer "F.Cu") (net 10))
 (segment (start 93.345 105.39) (end 87.015 99.06) (width 0.25) (layer "F.Cu") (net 10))
 (segment (start 86.36 81.28) (end 86.36 99.06) (width 0.25) (layer "B.Cu") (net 10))
 (segment (start 90.805 76.835) (end 86.36 81.28) (width 0.25) (layer "B.Cu") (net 10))
 (segment (start 93.67 60.655) (end 93.98 60.345) (width 0.25) (layer "F.Cu") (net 1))
 (segment (start 82.22 60.655) (end 80.01 62.865) (width 0.25) (layer "F.Cu") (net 1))
 (segment (start 87.09 60.655) (end 93.67 60.655) (width 0.25) (layer "F.Cu") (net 1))
 (segment (start 80.01 62.865) (end 80.01 73.66) (width 0.25) (layer "F.Cu") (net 1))
 (segment (start 87.09 60.655) (end 82.22 60.655) (width 0.25) (layer "F.Cu") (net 1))
 (segment (start 80.01 73.66) (end 83.185 76.835) (width 0.25) (layer "F.Cu") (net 1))
 (segment (start 87.09 63.155) (end 93.67 63.155) (width 0.25) (layer "F.Cu") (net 2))
 (segment (start 93.67 63.155) (end 93.98 62.845) (width 0.25) (layer "F.Cu") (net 2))
 (segment (start 81.28 66.04) (end 81.28 82.55) (width 0.25) (layer "B.Cu") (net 2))
 (segment (start 87.09 63.155) (end 84.165 63.155) (width 0.25) (layer "B.Cu") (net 2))
 (segment (start 81.28 82.55) (end 83.185 84.455) (width 0.25) (layer "B.Cu") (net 2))
 (segment (start 84.165 63.155) (end 81.28 66.04) (width 0.25) (layer "B.Cu") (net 2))
 (segment (start 80.645 92.075) (end 82.55 93.98) (width 0.25) (layer "F.Cu") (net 4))
 (segment (start 82.405 78.25) (end 80.645 80.01) (width 0.25) (layer "F.Cu") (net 4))
 (segment (start 93.345 100.33) (end 116.205 100.33) (width 0.25) (layer "F.Cu") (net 4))
 (segment (start 84.31 77.590991) (end 83.650991 78.25) (width 0.25) (layer "F.Cu") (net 4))
 (segment (start 83.650991 78.25) (end 82.405 78.25) (width 0.25) (layer "F.Cu") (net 4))
 (segment (start 80.645 80.01) (end 80.645 92.075) (width 0.25) (layer "F.Cu") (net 4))
 (segment (start 84.31 75.42) (end 84.31 77.590991) (width 0.25) (layer "F.Cu") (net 4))
 (segment (start 83.185 74.295) (end 84.31 75.42) (width 0.25) (layer "F.Cu") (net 4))
 (segment (start 116.205 100.33) (end 117.475 99.06) (width 0.25) (layer "F.Cu") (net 4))
 (segment (start 86.995 93.98) (end 93.345 100.33) (width 0.25) (layer "F.Cu") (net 4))
 (segment (start 82.55 93.98) (end 86.995 93.98) (width 0.25) (layer "F.Cu") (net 4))
 (segment (start 117.475 96.52) (end 114.935 96.52) (width 0.25) (layer "F.Cu") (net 6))
 (segment (start 92.71 92.075) (end 90.805 92.075) (width 0.25) (layer "F.Cu") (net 6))
 (segment (start 85.725 86.995) (end 83.185 86.995) (width 0.25) (layer "F.Cu") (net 6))
 (segment (start 113.665 95.25) (end 95.885 95.25) (width 0.25) (layer "F.Cu") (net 6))
 (segment (start 95.885 95.25) (end 92.71 92.075) (width 0.25) (layer "F.Cu") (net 6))
 (segment (start 114.935 96.52) (end 113.665 95.25) (width 0.25) (layer "F.Cu") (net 6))
 (segment (start 90.805 92.075) (end 85.725 86.995) (width 0.25) (layer "F.Cu") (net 6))
 (segment (start 90.805 86.995) (end 96.703875 92.893875) (width 0.25) (layer "F.Cu") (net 8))
 (segment (start 96.704749 92.893) (end 116.388 92.893) (width 0.25) (layer "F.Cu") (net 8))
 (segment (start 116.388 92.893) (end 117.475 93.98) (width 0.25) (layer "F.Cu") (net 8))
 (segment (start 96.703875 92.893875) (end 96.704749 92.893) (width 0.25) (layer "F.Cu") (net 8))
 (segment (start 90.805 74.295) (end 96.703875 80.193875) (width 0.25) (layer "B.Cu") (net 11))
 (segment (start 96.703875 80.193875) (end 96.704749 80.193) (width 0.25) (layer "B.Cu") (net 11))
 (segment (start 106.228 80.193) (end 117.475 91.44) (width 0.25) (layer "B.Cu") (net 11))
 (segment (start 96.704749 80.193) (end 106.228 80.193) (width 0.25) (layer "B.Cu") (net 11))
 (segment (start 123.825 73.66) (end 118.745 78.74) (width 0.25) (layer "F.Cu") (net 28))
 (segment (start 117.475 88.9) (end 116.388 87.813) (width 0.25) (layer "F.Cu") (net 28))
 (segment (start 116.388 87.813) (end 116.388 80.462) (width 0.25) (layer "F.Cu") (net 28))
 (segment (start 116.388 80.462) (end 117.023 79.827) (width 0.25) (layer "F.Cu") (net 28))
 (segment (start 118.293 79.827) (end 118.745 79.375) (width 0.25) (layer "F.Cu") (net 28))
 (segment (start 118.745 79.375) (end 118.745 78.74) (width 0.25) (layer "F.Cu") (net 28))
 (segment (start 117.023 79.827) (end 118.293 79.827) (width 0.25) (layer "F.Cu") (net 28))
 (segment (start 117.475 86.36) (end 123.825 86.36) (width 0.25) (layer "B.Cu") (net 29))
 (segment (start 118.89 85.235) (end 130.32 85.235) (width 0.25) (layer "F.Cu") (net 30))
 (segment (start 130.32 85.235) (end 131.445 86.36) (width 0.25) (layer "F.Cu") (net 30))
 (segment (start 117.475 83.82) (end 118.89 85.235) (width 0.25) (layer "F.Cu") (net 30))
 (segment (start 121.285 77.47) (end 117.475 81.28) (width 0.25) (layer "F.Cu") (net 31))
 (segment (start 131.445 73.66) (end 128.27 73.66) (width 0.25) (layer "F.Cu") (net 31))
 (segment (start 128.27 73.66) (end 124.46 77.47) (width 0.25) (layer "F.Cu") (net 31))
 (segment (start 124.46 77.47) (end 121.285 77.47) (width 0.25) (layer "F.Cu") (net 31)))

